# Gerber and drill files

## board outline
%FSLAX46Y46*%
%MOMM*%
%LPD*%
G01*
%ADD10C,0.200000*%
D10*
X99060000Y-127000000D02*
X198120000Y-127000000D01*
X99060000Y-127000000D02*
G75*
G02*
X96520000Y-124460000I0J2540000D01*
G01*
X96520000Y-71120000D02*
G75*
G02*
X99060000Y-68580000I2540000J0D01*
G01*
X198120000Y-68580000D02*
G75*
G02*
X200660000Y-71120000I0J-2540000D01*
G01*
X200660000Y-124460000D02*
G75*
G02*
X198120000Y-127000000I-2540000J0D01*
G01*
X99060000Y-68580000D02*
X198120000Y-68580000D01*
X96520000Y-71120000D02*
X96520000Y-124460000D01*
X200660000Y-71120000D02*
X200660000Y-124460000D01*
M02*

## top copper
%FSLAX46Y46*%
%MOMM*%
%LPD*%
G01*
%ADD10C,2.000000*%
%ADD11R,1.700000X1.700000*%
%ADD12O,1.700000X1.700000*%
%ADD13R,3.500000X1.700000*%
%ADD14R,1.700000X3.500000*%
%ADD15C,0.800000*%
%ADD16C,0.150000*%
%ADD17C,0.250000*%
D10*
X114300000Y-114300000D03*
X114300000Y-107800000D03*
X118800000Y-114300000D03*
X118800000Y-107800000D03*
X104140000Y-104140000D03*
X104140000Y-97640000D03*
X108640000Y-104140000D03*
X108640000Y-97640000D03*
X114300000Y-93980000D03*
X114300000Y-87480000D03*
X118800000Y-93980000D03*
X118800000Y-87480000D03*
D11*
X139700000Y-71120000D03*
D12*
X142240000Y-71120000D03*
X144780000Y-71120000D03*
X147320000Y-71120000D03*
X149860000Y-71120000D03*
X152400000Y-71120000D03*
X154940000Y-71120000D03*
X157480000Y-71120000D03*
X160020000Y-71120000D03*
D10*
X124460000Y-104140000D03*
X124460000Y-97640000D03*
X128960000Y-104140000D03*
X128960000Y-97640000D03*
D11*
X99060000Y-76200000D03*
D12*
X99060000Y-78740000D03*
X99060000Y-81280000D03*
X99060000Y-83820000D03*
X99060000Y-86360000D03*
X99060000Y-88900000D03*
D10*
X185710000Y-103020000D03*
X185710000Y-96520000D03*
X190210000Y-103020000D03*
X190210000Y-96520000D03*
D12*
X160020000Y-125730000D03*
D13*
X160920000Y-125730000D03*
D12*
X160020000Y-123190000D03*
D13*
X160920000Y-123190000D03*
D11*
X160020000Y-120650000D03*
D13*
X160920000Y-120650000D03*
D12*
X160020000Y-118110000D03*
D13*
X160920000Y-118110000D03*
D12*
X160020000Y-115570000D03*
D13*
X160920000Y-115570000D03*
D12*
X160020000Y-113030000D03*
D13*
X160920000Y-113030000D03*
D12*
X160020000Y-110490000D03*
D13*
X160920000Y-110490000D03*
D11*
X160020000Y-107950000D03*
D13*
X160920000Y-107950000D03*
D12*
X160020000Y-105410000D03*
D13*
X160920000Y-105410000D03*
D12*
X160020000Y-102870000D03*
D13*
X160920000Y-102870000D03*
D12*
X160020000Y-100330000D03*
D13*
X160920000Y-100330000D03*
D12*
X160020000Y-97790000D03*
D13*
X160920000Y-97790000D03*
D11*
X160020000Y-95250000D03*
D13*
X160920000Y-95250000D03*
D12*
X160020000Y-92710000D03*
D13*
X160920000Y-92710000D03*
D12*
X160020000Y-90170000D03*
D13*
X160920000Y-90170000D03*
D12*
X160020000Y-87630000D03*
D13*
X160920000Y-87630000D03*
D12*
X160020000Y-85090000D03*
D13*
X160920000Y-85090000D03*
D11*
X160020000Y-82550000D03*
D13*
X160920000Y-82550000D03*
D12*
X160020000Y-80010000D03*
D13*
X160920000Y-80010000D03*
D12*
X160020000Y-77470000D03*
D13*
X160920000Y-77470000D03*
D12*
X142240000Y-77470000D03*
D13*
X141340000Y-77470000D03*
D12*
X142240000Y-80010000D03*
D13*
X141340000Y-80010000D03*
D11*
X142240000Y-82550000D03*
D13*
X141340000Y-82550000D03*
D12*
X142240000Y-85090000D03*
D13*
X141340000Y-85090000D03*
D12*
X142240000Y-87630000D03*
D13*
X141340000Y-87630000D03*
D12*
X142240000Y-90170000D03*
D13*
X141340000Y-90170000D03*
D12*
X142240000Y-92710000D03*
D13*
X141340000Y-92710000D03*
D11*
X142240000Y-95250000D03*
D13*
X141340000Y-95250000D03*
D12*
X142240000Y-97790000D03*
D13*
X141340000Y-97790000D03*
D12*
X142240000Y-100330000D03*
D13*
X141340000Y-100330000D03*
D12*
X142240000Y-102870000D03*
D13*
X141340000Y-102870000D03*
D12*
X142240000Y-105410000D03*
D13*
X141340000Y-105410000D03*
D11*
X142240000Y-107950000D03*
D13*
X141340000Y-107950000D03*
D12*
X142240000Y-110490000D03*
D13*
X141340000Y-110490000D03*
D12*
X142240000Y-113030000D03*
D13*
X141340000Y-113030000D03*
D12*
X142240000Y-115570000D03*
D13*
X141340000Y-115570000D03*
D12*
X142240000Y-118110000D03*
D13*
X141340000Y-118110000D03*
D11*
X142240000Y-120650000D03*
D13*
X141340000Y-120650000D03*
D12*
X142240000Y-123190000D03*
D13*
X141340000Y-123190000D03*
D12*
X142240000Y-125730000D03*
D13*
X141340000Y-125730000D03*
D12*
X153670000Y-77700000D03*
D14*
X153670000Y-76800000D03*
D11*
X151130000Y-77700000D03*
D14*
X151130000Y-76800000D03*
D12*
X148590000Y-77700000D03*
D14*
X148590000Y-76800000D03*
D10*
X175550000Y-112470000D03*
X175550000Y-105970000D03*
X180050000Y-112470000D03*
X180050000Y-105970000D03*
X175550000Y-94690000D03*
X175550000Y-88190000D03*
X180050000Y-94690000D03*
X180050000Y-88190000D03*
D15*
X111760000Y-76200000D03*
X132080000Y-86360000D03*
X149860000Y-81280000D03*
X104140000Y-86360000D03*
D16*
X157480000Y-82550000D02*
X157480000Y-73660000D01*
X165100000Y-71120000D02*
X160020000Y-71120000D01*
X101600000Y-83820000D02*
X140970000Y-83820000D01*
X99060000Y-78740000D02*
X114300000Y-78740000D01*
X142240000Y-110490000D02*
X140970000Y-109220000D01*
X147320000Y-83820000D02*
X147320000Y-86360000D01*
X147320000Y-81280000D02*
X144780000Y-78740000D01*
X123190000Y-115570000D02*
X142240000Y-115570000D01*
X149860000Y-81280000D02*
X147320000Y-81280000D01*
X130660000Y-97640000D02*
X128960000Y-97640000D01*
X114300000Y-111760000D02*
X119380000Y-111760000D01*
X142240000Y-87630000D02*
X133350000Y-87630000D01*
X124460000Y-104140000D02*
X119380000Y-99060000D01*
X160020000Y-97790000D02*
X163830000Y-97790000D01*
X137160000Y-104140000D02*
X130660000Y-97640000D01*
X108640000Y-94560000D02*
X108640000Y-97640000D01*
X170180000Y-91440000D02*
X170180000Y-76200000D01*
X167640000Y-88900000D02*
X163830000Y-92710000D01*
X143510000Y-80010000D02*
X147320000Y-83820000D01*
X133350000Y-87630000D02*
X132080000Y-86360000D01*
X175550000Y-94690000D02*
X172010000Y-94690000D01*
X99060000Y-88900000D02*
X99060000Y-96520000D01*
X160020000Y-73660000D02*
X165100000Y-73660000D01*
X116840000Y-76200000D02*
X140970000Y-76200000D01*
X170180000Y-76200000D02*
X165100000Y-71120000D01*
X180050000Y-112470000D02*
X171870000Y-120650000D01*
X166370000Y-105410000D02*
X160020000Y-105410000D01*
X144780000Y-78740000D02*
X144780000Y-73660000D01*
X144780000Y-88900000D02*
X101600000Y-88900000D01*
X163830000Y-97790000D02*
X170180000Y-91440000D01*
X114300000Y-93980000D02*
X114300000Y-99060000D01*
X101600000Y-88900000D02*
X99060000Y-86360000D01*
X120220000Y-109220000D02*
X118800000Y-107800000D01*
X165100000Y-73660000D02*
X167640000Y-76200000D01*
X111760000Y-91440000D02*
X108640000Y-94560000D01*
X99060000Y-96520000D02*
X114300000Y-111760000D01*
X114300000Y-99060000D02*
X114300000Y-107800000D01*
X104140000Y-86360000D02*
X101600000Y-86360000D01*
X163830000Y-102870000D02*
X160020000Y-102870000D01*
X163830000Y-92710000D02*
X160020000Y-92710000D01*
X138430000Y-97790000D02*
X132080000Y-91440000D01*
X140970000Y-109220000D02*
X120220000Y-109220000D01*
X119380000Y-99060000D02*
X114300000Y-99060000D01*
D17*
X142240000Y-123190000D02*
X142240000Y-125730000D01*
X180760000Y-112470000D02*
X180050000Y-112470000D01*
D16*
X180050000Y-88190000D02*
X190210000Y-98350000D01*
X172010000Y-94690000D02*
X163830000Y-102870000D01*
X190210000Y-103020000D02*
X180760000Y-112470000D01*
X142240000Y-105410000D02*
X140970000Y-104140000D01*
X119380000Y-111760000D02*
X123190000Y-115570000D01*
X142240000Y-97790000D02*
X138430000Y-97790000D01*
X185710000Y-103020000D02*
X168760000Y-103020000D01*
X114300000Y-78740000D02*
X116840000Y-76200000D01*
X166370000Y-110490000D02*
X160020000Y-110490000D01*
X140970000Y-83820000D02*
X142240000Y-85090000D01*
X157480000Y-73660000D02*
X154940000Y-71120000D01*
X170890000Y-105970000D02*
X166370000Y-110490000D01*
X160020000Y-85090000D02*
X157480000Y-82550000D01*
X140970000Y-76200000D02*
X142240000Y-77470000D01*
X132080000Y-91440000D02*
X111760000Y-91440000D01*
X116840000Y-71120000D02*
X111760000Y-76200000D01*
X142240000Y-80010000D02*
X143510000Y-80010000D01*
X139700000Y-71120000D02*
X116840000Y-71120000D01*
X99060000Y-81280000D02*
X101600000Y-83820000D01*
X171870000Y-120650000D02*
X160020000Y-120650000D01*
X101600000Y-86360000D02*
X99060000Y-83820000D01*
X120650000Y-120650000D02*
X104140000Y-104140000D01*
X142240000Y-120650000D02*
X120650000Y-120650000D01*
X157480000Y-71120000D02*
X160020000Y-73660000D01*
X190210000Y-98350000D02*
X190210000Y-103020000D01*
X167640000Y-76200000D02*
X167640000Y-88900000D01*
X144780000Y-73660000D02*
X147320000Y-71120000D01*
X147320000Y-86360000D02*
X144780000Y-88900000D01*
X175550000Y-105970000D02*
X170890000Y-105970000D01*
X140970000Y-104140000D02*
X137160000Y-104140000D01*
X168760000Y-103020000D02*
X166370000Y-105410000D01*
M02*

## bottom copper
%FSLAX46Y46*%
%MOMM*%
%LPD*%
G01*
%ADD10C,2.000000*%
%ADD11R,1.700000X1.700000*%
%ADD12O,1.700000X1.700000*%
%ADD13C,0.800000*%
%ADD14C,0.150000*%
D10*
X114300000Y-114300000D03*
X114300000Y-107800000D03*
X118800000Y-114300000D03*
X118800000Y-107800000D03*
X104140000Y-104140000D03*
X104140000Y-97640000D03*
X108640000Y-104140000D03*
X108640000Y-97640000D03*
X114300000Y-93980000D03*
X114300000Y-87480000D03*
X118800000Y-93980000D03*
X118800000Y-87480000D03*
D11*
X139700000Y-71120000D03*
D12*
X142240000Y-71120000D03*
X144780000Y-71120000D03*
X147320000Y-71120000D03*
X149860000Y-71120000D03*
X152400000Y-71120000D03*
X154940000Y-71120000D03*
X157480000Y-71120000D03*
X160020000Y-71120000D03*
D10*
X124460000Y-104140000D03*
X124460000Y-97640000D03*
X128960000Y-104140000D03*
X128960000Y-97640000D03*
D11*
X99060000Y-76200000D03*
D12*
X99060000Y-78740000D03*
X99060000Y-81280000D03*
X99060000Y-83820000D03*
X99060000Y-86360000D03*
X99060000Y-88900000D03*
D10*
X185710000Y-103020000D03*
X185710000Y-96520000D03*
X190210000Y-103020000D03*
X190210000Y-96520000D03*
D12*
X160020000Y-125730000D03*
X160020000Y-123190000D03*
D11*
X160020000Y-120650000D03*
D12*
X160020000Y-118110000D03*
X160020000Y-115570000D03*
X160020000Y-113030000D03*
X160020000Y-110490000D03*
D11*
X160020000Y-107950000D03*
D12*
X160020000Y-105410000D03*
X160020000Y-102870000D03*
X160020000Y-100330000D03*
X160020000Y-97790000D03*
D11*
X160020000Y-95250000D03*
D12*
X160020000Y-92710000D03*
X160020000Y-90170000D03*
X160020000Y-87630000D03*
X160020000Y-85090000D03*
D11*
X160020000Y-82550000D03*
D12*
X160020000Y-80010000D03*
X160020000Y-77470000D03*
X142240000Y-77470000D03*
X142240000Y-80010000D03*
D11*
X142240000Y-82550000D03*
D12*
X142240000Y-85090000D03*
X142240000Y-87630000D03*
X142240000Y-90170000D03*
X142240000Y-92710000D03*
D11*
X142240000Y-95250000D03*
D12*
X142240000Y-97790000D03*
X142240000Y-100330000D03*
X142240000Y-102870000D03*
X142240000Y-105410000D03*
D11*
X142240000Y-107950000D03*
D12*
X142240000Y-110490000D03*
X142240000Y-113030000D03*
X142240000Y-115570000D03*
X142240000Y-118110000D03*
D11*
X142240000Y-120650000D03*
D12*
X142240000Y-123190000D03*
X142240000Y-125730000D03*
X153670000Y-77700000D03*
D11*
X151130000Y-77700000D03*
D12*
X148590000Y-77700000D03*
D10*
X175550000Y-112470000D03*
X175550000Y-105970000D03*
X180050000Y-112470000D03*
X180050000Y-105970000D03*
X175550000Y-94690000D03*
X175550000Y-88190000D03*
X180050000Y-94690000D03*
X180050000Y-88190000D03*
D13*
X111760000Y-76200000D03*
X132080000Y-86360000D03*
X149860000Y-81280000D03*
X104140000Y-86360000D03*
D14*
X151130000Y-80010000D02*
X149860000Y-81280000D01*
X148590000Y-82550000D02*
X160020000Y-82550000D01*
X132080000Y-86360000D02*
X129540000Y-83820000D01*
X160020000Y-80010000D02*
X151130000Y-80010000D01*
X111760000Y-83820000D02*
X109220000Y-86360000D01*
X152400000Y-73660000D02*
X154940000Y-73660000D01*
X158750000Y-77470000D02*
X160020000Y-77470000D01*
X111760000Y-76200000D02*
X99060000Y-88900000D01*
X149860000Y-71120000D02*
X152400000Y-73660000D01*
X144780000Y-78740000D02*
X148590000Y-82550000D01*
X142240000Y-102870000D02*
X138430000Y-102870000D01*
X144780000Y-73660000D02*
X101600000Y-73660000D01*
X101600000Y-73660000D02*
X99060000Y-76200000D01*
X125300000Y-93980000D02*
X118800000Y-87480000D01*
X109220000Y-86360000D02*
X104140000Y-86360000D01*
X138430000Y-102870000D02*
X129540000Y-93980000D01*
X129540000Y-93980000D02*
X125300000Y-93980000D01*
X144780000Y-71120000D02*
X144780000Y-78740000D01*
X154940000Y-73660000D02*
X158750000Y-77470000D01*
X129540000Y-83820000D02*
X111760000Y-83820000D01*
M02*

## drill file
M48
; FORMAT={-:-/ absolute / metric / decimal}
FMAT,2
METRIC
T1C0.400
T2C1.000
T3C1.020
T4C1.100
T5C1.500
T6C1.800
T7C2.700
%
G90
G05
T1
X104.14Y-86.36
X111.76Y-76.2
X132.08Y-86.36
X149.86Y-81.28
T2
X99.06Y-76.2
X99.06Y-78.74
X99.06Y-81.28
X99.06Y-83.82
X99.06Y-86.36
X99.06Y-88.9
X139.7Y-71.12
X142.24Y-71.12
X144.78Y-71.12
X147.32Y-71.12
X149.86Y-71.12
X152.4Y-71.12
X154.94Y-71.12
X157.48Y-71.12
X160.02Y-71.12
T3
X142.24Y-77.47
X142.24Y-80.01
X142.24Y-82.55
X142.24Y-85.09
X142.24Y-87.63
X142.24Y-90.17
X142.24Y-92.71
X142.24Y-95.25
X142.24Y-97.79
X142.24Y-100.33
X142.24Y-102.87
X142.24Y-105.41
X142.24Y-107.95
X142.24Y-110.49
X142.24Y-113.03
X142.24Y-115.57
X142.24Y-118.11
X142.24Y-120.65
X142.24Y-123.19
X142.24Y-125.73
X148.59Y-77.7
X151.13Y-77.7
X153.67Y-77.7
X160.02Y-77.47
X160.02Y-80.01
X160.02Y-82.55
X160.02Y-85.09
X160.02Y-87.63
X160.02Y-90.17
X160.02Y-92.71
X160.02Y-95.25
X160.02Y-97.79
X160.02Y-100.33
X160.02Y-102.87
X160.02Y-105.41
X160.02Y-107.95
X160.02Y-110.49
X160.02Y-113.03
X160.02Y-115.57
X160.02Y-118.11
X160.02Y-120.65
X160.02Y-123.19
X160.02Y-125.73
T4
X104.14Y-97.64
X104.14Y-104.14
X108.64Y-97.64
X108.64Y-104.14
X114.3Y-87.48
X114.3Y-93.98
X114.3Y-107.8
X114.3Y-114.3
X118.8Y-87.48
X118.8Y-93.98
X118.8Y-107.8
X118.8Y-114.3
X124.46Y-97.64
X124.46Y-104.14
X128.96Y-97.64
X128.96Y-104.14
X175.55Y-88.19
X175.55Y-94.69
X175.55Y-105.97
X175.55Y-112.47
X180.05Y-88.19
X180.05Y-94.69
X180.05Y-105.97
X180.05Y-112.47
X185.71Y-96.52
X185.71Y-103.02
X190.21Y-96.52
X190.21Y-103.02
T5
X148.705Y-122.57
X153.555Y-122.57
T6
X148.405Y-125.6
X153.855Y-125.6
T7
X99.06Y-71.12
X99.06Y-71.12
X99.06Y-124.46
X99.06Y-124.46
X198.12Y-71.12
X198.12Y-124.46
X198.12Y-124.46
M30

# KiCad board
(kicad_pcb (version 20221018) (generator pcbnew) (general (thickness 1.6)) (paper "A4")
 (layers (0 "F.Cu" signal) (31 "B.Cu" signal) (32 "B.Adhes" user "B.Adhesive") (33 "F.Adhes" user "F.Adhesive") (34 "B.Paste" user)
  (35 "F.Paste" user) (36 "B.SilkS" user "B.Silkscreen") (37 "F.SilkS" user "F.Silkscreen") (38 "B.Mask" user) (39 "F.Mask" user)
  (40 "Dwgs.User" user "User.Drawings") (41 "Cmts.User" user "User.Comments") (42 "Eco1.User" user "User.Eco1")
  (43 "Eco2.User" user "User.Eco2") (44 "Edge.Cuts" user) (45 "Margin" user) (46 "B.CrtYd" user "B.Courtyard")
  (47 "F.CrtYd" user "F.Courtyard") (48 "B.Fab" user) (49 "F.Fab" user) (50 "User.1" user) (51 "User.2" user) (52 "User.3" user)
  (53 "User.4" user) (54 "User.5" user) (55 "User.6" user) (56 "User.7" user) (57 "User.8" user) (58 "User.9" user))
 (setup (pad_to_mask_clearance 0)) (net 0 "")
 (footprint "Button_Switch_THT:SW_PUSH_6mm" (layer "F.Cu") (at 114.3 114.3 90)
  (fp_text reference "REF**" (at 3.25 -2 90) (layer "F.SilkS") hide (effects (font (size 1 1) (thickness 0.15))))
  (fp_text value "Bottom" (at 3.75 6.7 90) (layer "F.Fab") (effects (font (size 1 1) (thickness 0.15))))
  (pad "1" thru_hole circle (at 0 0 180) (size 2 2) (drill 1.1) (layers "*.Cu" "*.Mask"))
  (pad "1" thru_hole circle (at 6.5 0 180) (size 2 2) (drill 1.1) (layers "*.Cu" "*.Mask"))
  (pad "2" thru_hole circle (at 0 4.5 180) (size 2 2) (drill 1.1) (layers "*.Cu" "*.Mask"))
  (pad "2" thru_hole circle (at 6.5 4.5 180) (size 2 2) (drill 1.1) (layers "*.Cu" "*.Mask")))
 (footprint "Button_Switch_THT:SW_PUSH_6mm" (layer "F.Cu") (at 104.14 104.14 90)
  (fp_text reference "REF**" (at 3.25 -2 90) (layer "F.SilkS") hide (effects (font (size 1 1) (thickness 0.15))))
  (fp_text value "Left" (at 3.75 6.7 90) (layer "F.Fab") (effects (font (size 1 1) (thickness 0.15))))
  (pad "1" thru_hole circle (at 0 0 180) (size 2 2) (drill 1.1) (layers "*.Cu" "*.Mask"))
  (pad "1" thru_hole circle (at 6.5 0 180) (size 2 2) (drill 1.1) (layers "*.Cu" "*.Mask"))
  (pad "2" thru_hole circle (at 0 4.5 180) (size 2 2) (drill 1.1) (layers "*.Cu" "*.Mask"))
  (pad "2" thru_hole circle (at 6.5 4.5 180) (size 2 2) (drill 1.1) (layers "*.Cu" "*.Mask")))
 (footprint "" (layer "F.Cu") (at 198.12 71.12)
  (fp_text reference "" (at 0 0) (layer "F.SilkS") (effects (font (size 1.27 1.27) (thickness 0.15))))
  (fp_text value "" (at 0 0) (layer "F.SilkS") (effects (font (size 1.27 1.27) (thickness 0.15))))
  (pad "" np_thru_hole circle (at 0 0) (size 2.7 2.7) (drill 2.7) (layers "F&B.Cu" "*.Mask")))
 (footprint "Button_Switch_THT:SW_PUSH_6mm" (layer "F.Cu") (at 114.3 93.98 90)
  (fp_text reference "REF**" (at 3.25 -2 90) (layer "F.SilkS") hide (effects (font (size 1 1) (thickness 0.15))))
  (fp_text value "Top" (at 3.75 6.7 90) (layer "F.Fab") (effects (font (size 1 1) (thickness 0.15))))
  (pad "1" thru_hole circle (at 0 0 180) (size 2 2) (drill 1.1) (layers "*.Cu" "*.Mask"))
  (pad "1" thru_hole circle (at 6.5 0 180) (size 2 2) (drill 1.1) (layers "*.Cu" "*.Mask"))
  (pad "2" thru_hole circle (at 0 4.5 180) (size 2 2) (drill 1.1) (layers "*.Cu" "*.Mask"))
  (pad "2" thru_hole circle (at 6.5 4.5 180) (size 2 2) (drill 1.1) (layers "*.Cu" "*.Mask")))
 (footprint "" (layer "F.Cu") (at 99.06 71.12)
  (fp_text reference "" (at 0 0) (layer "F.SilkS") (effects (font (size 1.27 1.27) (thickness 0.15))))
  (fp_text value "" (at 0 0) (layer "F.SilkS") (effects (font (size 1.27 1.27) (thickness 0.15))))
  (pad "" np_thru_hole circle (at 0 0) (size 2.7 2.7) (drill 2.7) (layers "F&B.Cu" "*.Mask")))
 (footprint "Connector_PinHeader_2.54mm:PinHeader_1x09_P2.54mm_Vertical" (layer "F.Cu") (at 139.7 71.12 90)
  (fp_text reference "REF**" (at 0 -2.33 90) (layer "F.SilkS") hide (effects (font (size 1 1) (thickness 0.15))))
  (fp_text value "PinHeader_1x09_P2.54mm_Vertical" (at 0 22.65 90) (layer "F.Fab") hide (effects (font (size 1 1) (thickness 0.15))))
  (pad "1" thru_hole rect (at 0 0 90) (size 1.7 1.7) (drill 1) (layers "*.Cu" "*.Mask"))
  (pad "2" thru_hole oval (at 0 2.54 90) (size 1.7 1.7) (drill 1) (layers "*.Cu" "*.Mask"))
  (pad "3" thru_hole oval (at 0 5.08 90) (size 1.7 1.7) (drill 1) (layers "*.Cu" "*.Mask"))
  (pad "4" thru_hole oval (at 0 7.62 90) (size 1.7 1.7) (drill 1) (layers "*.Cu" "*.Mask"))
  (pad "5" thru_hole oval (at 0 10.16 90) (size 1.7 1.7) (drill 1) (layers "*.Cu" "*.Mask"))
  (pad "6" thru_hole oval (at 0 12.7 90) (size 1.7 1.7) (drill 1) (layers "*.Cu" "*.Mask"))
  (pad "7" thru_hole oval (at 0 15.24 90) (size 1.7 1.7) (drill 1) (layers "*.Cu" "*.Mask"))
  (pad "8" thru_hole oval (at 0 17.78 90) (size 1.7 1.7) (drill 1) (layers "*.Cu" "*.Mask"))
  (pad "9" thru_hole oval (at 0 20.32 90) (size 1.7 1.7) (drill 1) (layers "*.Cu" "*.Mask")))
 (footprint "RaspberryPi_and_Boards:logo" (layer "F.Cu") (at 190.5 76.2)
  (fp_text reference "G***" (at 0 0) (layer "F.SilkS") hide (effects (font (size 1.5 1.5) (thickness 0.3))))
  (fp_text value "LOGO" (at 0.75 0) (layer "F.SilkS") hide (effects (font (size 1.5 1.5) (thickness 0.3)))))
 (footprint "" (layer "F.Cu") (at 198.12 124.46)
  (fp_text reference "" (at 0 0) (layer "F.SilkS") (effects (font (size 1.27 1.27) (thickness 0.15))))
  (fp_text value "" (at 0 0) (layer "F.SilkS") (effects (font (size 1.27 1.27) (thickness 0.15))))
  (pad "" np_thru_hole circle (at 0 0) (size 2.7 2.7) (drill 2.7) (layers "F&B.Cu" "*.Mask")))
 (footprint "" (layer "F.Cu") (at 198.12 124.46)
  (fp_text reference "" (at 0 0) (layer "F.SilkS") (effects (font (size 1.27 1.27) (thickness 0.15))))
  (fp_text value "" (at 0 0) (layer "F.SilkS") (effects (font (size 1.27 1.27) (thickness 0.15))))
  (pad "" np_thru_hole circle (at 0 0) (size 2.7 2.7) (drill 2.7) (layers "F&B.Cu" "*.Mask")))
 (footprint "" (layer "F.Cu") (at 99.06 124.46)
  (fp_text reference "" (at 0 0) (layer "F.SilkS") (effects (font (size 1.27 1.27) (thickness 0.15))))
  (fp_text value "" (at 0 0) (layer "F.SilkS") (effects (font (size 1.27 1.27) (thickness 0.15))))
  (pad "" np_thru_hole circle (at 0 0) (size 2.7 2.7) (drill 2.7) (layers "F&B.Cu" "*.Mask")))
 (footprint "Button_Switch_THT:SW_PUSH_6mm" (layer "F.Cu") (at 124.46 104.14 90)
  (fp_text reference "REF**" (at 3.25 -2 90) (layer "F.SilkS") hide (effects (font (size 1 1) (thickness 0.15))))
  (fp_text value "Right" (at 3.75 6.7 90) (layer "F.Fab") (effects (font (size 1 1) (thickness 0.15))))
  (pad "1" thru_hole circle (at 0 0 180) (size 2 2) (drill 1.1) (layers "*.Cu" "*.Mask"))
  (pad "1" thru_hole circle (at 6.5 0 180) (size 2 2) (drill 1.1) (layers "*.Cu" "*.Mask"))
  (pad "2" thru_hole circle (at 0 4.5 180) (size 2 2) (drill 1.1) (layers "*.Cu" "*.Mask"))
  (pad "2" thru_hole circle (at 6.5 4.5 180) (size 2 2) (drill 1.1) (layers "*.Cu" "*.Mask")))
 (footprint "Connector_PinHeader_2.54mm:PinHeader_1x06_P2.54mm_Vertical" (layer "F.Cu") (at 99.06 76.2)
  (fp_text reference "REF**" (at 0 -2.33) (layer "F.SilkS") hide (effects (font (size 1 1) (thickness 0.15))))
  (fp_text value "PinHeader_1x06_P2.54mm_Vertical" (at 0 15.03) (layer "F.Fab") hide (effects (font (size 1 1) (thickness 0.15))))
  (pad "1" thru_hole rect (at 0 0) (size 1.7 1.7) (drill 1) (layers "*.Cu" "*.Mask"))
  (pad "2" thru_hole oval (at 0 2.54) (size 1.7 1.7) (drill 1) (layers "*.Cu" "*.Mask"))
  (pad "3" thru_hole oval (at 0 5.08) (size 1.7 1.7) (drill 1) (layers "*.Cu" "*.Mask"))
  (pad "4" thru_hole oval (at 0 7.62) (size 1.7 1.7) (drill 1) (layers "*.Cu" "*.Mask"))
  (pad "5" thru_hole oval (at 0 10.16) (size 1.7 1.7) (drill 1) (layers "*.Cu" "*.Mask"))
  (pad "6" thru_hole oval (at 0 12.7) (size 1.7 1.7) (drill 1) (layers "*.Cu" "*.Mask")))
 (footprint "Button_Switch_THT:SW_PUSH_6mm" (layer "F.Cu") (at 185.71 103.02 90)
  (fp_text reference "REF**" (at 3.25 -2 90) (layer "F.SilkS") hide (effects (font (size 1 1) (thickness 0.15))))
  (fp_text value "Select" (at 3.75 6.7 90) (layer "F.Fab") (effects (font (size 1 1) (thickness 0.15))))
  (pad "1" thru_hole circle (at 0 0 180) (size 2 2) (drill 1.1) (layers "*.Cu" "*.Mask"))
  (pad "1" thru_hole circle (at 6.5 0 180) (size 2 2) (drill 1.1) (layers "*.Cu" "*.Mask"))
  (pad "2" thru_hole circle (at 0 4.5 180) (size 2 2) (drill 1.1) (layers "*.Cu" "*.Mask"))
  (pad "2" thru_hole circle (at 6.5 4.5 180) (size 2 2) (drill 1.1) (layers "*.Cu" "*.Mask")))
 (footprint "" (layer "F.Cu") (at 99.06 124.46)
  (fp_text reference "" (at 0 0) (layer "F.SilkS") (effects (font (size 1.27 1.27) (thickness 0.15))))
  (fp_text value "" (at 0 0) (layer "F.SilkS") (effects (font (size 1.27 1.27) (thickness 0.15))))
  (pad "" np_thru_hole circle (at 0 0) (size 2.7 2.7) (drill 2.7) (layers "F&B.Cu" "*.Mask")))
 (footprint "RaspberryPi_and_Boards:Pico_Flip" (layer "F.Cu") (at 151.13 101.6 180)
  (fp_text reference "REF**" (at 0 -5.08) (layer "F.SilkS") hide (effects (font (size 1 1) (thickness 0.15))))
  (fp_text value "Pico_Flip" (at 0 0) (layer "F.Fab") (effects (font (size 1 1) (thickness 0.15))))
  (pad "" np_thru_hole oval (at -2.725 -24 180) (size 1.8 1.8) (drill 1.8) (layers "*.Cu" "*.Mask"))
  (pad "" np_thru_hole oval (at -2.425 -20.97 180) (size 1.5 1.5) (drill 1.5) (layers "*.Cu" "*.Mask"))
  (pad "" np_thru_hole oval (at 2.425 -20.97 180) (size 1.5 1.5) (drill 1.5) (layers "*.Cu" "*.Mask"))
  (pad "" np_thru_hole oval (at 2.725 -24 180) (size 1.8 1.8) (drill 1.8) (layers "*.Cu" "*.Mask"))
  (pad "1" thru_hole oval (at -8.89 -24.13 180) (size 1.7 1.7) (drill 1.02) (layers "*.Cu" "*.Mask"))
  (pad "1" smd rect (at -8.89 -24.13 180) (size 3.5 1.7) (drill (offset -0.9 0)) (layers "F.Cu" "F.Mask"))
  (pad "2" thru_hole oval (at -8.89 -21.59 180) (size 1.7 1.7) (drill 1.02) (layers "*.Cu" "*.Mask"))
  (pad "2" smd rect (at -8.89 -21.59 180) (size 3.5 1.7) (drill (offset -0.9 0)) (layers "F.Cu" "F.Mask"))
  (pad "3" thru_hole rect (at -8.89 -19.05 180) (size 1.7 1.7) (drill 1.02) (layers "*.Cu" "*.Mask"))
  (pad "3" smd rect (at -8.89 -19.05 180) (size 3.5 1.7) (drill (offset -0.9 0)) (layers "F.Cu" "F.Mask"))
  (pad "4" thru_hole oval (at -8.89 -16.51 180) (size 1.7 1.7) (drill 1.02) (layers "*.Cu" "*.Mask"))
  (pad "4" smd rect (at -8.89 -16.51 180) (size 3.5 1.7) (drill (offset -0.9 0)) (layers "F.Cu" "F.Mask"))
  (pad "5" thru_hole oval (at -8.89 -13.97 180) (size 1.7 1.7) (drill 1.02) (layers "*.Cu" "*.Mask"))
  (pad "5" smd rect (at -8.89 -13.97 180) (size 3.5 1.7) (drill (offset -0.9 0)) (layers "F.Cu" "F.Mask"))
  (pad "6" thru_hole oval (at -8.89 -11.43 180) (size 1.7 1.7) (drill 1.02) (layers "*.Cu" "*.Mask"))
  (pad "6" smd rect (at -8.89 -11.43 180) (size 3.5 1.7) (drill (offset -0.9 0)) (layers "F.Cu" "F.Mask"))
  (pad "7" thru_hole oval (at -8.89 -8.89 180) (size 1.7 1.7) (drill 1.02) (layers "*.Cu" "*.Mask"))
  (pad "7" smd rect (at -8.89 -8.89 180) (size 3.5 1.7) (drill (offset -0.9 0)) (layers "F.Cu" "F.Mask"))
  (pad "8" thru_hole rect (at -8.89 -6.35 180) (size 1.7 1.7) (drill 1.02) (layers "*.Cu" "*.Mask"))
  (pad "8" smd rect (at -8.89 -6.35 180) (size 3.5 1.7) (drill (offset -0.9 0)) (layers "F.Cu" "F.Mask"))
  (pad "9" thru_hole oval (at -8.89 -3.81 180) (size 1.7 1.7) (drill 1.02) (layers "*.Cu" "*.Mask"))
  (pad "9" smd rect (at -8.89 -3.81 180) (size 3.5 1.7) (drill (offset -0.9 0)) (layers "F.Cu" "F.Mask"))
  (pad "10" thru_hole oval (at -8.89 -1.27 180) (size 1.7 1.7) (drill 1.02) (layers "*.Cu" "*.Mask"))
  (pad "10" smd rect (at -8.89 -1.27 180) (size 3.5 1.7) (drill (offset -0.9 0)) (layers "F.Cu" "F.Mask"))
  (pad "11" thru_hole oval (at -8.89 1.27 180) (size 1.7 1.7) (drill 1.02) (layers "*.Cu" "*.Mask"))
  (pad "11" smd rect (at -8.89 1.27 180) (size 3.5 1.7) (drill (offset -0.9 0)) (layers "F.Cu" "F.Mask"))
  (pad "12" thru_hole oval (at -8.89 3.81 180) (size 1.7 1.7) (drill 1.02) (layers "*.Cu" "*.Mask"))
  (pad "12" smd rect (at -8.89 3.81 180) (size 3.5 1.7) (drill (offset -0.9 0)) (layers "F.Cu" "F.Mask"))
  (pad "13" thru_hole rect (at -8.89 6.35 180) (size 1.7 1.7) (drill 1.02) (layers "*.Cu" "*.Mask"))
  (pad "13" smd rect (at -8.89 6.35 180) (size 3.5 1.7) (drill (offset -0.9 0)) (layers "F.Cu" "F.Mask"))
  (pad "14" thru_hole oval (at -8.89 8.89 180) (size 1.7 1.7) (drill 1.02) (layers "*.Cu" "*.Mask"))
  (pad "14" smd rect (at -8.89 8.89 180) (size 3.5 1.7) (drill (offset -0.9 0)) (layers "F.Cu" "F.Mask"))
  (pad "15" thru_hole oval (at -8.89 11.43 180) (size 1.7 1.7) (drill 1.02) (layers "*.Cu" "*.Mask"))
  (pad "15" smd rect (at -8.89 11.43 180) (size 3.5 1.7) (drill (offset -0.9 0)) (layers "F.Cu" "F.Mask"))
  (pad "16" thru_hole oval (at -8.89 13.97 180) (size 1.7 1.7) (drill 1.02) (layers "*.Cu" "*.Mask"))
  (pad "16" smd rect (at -8.89 13.97 180) (size 3.5 1.7) (drill (offset -0.9 0)) (layers "F.Cu" "F.Mask"))
  (pad "17" thru_hole oval (at -8.89 16.51 180) (size 1.7 1.7) (drill 1.02) (layers "*.Cu" "*.Mask"))
  (pad "17" smd rect (at -8.89 16.51 180) (size 3.5 1.7) (drill (offset -0.9 0)) (layers "F.Cu" "F.Mask"))
  (pad "18" thru_hole rect (at -8.89 19.05 180) (size 1.7 1.7) (drill 1.02) (layers "*.Cu" "*.Mask"))
  (pad "18" smd rect (at -8.89 19.05 180) (size 3.5 1.7) (drill (offset -0.9 0)) (layers "F.Cu" "F.Mask"))
  (pad "19" thru_hole oval (at -8.89 21.59 180) (size 1.7 1.7) (drill 1.02) (layers "*.Cu" "*.Mask"))
  (pad "19" smd rect (at -8.89 21.59 180) (size 3.5 1.7) (drill (offset -0.9 0)) (layers "F.Cu" "F.Mask"))
  (pad "20" thru_hole oval (at -8.89 24.13 180) (size 1.7 1.7) (drill 1.02) (layers "*.Cu" "*.Mask"))
  (pad "20" smd rect (at -8.89 24.13 180) (size 3.5 1.7) (drill (offset -0.9 0)) (layers "F.Cu" "F.Mask"))
  (pad "21" thru_hole oval (at 8.89 24.13 180) (size 1.7 1.7) (drill 1.02) (layers "*.Cu" "*.Mask"))
  (pad "21" smd rect (at 8.89 24.13 180) (size 3.5 1.7) (drill (offset 0.9 0)) (layers "F.Cu" "F.Mask"))
  (pad "22" thru_hole oval (at 8.89 21.59 180) (size 1.7 1.7) (drill 1.02) (layers "*.Cu" "*.Mask"))
  (pad "22" smd rect (at 8.89 21.59 180) (size 3.5 1.7) (drill (offset 0.9 0)) (layers "F.Cu" "F.Mask"))
  (pad "23" thru_hole rect (at 8.89 19.05 180) (size 1.7 1.7) (drill 1.02) (layers "*.Cu" "*.Mask"))
  (pad "23" smd rect (at 8.89 19.05 180) (size 3.5 1.7) (drill (offset 0.9 0)) (layers "F.Cu" "F.Mask"))
  (pad "24" thru_hole oval (at 8.89 16.51 180) (size 1.7 1.7) (drill 1.02) (layers "*.Cu" "*.Mask"))
  (pad "24" smd rect (at 8.89 16.51 180) (size 3.5 1.7) (drill (offset 0.9 0)) (layers "F.Cu" "F.Mask"))
  (pad "25" thru_hole oval (at 8.89 13.97 180) (size 1.7 1.7) (drill 1.02) (layers "*.Cu" "*.Mask"))
  (pad "25" smd rect (at 8.89 13.97 180) (size 3.5 1.7) (drill (offset 0.9 0)) (layers "F.Cu" "F.Mask"))
  (pad "26" thru_hole oval (at 8.89 11.43 180) (size 1.7 1.7) (drill 1.02) (layers "*.Cu" "*.Mask"))
  (pad "26" smd rect (at 8.89 11.43 180) (size 3.5 1.7) (drill (offset 0.9 0)) (layers "F.Cu" "F.Mask"))
  (pad "27" thru_hole oval (at 8.89 8.89 180) (size 1.7 1.7) (drill 1.02) (layers "*.Cu" "*.Mask"))
  (pad "27" smd rect (at 8.89 8.89 180) (size 3.5 1.7) (drill (offset 0.9 0)) (layers "F.Cu" "F.Mask"))
  (pad "28" thru_hole rect (at 8.89 6.35 180) (size 1.7 1.7) (drill 1.02) (layers "*.Cu" "*.Mask"))
  (pad "28" smd rect (at 8.89 6.35 180) (size 3.5 1.7) (drill (offset 0.9 0)) (layers "F.Cu" "F.Mask"))
  (pad "29" thru_hole oval (at 8.89 3.81 180) (size 1.7 1.7) (drill 1.02) (layers "*.Cu" "*.Mask"))
  (pad "29" smd rect (at 8.89 3.81 180) (size 3.5 1.7) (drill (offset 0.9 0)) (layers "F.Cu" "F.Mask"))
  (pad "30" thru_hole oval (at 8.89 1.27 180) (size 1.7 1.7) (drill 1.02) (layers "*.Cu" "*.Mask"))
  (pad "30" smd rect (at 8.89 1.27 180) (size 3.5 1.7) (drill (offset 0.9 0)) (layers "F.Cu" "F.Mask"))
  (pad "31" thru_hole oval (at 8.89 -1.27 180) (size 1.7 1.7) (drill 1.02) (layers "*.Cu" "*.Mask"))
  (pad "31" smd rect (at 8.89 -1.27 180) (size 3.5 1.7) (drill (offset 0.9 0)) (layers "F.Cu" "F.Mask"))
  (pad "32" thru_hole oval (at 8.89 -3.81 180) (size 1.7 1.7) (drill 1.02) (layers "*.Cu" "*.Mask"))
  (pad "32" smd rect (at 8.89 -3.81 180) (size 3.5 1.7) (drill (offset 0.9 0)) (layers "F.Cu" "F.Mask"))
  (pad "33" thru_hole rect (at 8.89 -6.35 180) (size 1.7 1.7) (drill 1.02) (layers "*.Cu" "*.Mask"))
  (pad "33" smd rect (at 8.89 -6.35 180) (size 3.5 1.7) (drill (offset 0.9 0)) (layers "F.Cu" "F.Mask"))
  (pad "34" thru_hole oval (at 8.89 -8.89 180) (size 1.7 1.7) (drill 1.02) (layers "*.Cu" "*.Mask"))
  (pad "34" smd rect (at 8.89 -8.89 180) (size 3.5 1.7) (drill (offset 0.9 0)) (layers "F.Cu" "F.Mask"))
  (pad "35" thru_hole oval (at 8.89 -11.43 180) (size 1.7 1.7) (drill 1.02) (layers "*.Cu" "*.Mask"))
  (pad "35" smd rect (at 8.89 -11.43 180) (size 3.5 1.7) (drill (offset 0.9 0)) (layers "F.Cu" "F.Mask"))
  (pad "36" thru_hole oval (at 8.89 -13.97 180) (size 1.7 1.7) (drill 1.02) (layers "*.Cu" "*.Mask"))
  (pad "36" smd rect (at 8.89 -13.97 180) (size 3.5 1.7) (drill (offset 0.9 0)) (layers "F.Cu" "F.Mask"))
  (pad "37" thru_hole oval (at 8.89 -16.51 180) (size 1.7 1.7) (drill 1.02) (layers "*.Cu" "*.Mask"))
  (pad "37" smd rect (at 8.89 -16.51 180) (size 3.5 1.7) (drill (offset 0.9 0)) (layers "F.Cu" "F.Mask"))
  (pad "38" thru_hole rect (at 8.89 -19.05 180) (size 1.7 1.7) (drill 1.02) (layers "*.Cu" "*.Mask"))
  (pad "38" smd rect (at 8.89 -19.05 180) (size 3.5 1.7) (drill (offset 0.9 0)) (layers "F.Cu" "F.Mask"))
  (pad "39" thru_hole oval (at 8.89 -21.59 180) (size 1.7 1.7) (drill 1.02) (layers "*.Cu" "*.Mask"))
  (pad "39" smd rect (at 8.89 -21.59 180) (size 3.5 1.7) (drill (offset 0.9 0)) (layers "F.Cu" "F.Mask"))
  (pad "40" thru_hole oval (at 8.89 -24.13 180) (size 1.7 1.7) (drill 1.02) (layers "*.Cu" "*.Mask"))
  (pad "40" smd rect (at 8.89 -24.13 180) (size 3.5 1.7) (drill (offset 0.9 0)) (layers "F.Cu" "F.Mask"))
  (pad "41" thru_hole oval (at -2.54 23.9 180) (size 1.7 1.7) (drill 1.02) (layers "*.Cu" "*.Mask"))
  (pad "41" smd rect (at -2.54 23.9 270) (size 3.5 1.7) (drill (offset -0.9 0)) (layers "F.Cu" "F.Mask"))
  (pad "42" thru_hole rect (at 0 23.9 180) (size 1.7 1.7) (drill 1.02) (layers "*.Cu" "*.Mask"))
  (pad "42" smd rect (at 0 23.9 270) (size 3.5 1.7) (drill (offset -0.9 0)) (layers "F.Cu" "F.Mask"))
  (pad "43" thru_hole oval (at 2.54 23.9 180) (size 1.7 1.7) (drill 1.02) (layers "*.Cu" "*.Mask"))
  (pad "43" smd rect (at 2.54 23.9 270) (size 3.5 1.7) (drill (offset -0.9 0)) (layers "F.Cu" "F.Mask")))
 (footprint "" (layer "F.Cu") (at 99.06 71.12)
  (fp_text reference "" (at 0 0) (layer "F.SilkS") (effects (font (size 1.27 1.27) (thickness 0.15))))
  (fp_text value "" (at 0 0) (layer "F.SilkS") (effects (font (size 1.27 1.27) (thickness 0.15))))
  (pad "" np_thru_hole circle (at 0 0) (size 2.7 2.7) (drill 2.7) (layers "F&B.Cu" "*.Mask")))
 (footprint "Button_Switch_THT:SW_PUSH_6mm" (layer "F.Cu") (at 175.55 112.47 90)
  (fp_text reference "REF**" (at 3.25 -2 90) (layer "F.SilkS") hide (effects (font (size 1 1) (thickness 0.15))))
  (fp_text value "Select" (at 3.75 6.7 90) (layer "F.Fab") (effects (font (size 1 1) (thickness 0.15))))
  (pad "1" thru_hole circle (at 0 0 180) (size 2 2) (drill 1.1) (layers "*.Cu" "*.Mask"))
  (pad "1" thru_hole circle (at 6.5 0 180) (size 2 2) (drill 1.1) (layers "*.Cu" "*.Mask"))
  (pad "2" thru_hole circle (at 0 4.5 180) (size 2 2) (drill 1.1) (layers "*.Cu" "*.Mask"))
  (pad "2" thru_hole circle (at 6.5 4.5 180) (size 2 2) (drill 1.1) (layers "*.Cu" "*.Mask")))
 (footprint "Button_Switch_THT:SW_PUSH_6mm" (layer "F.Cu") (at 175.55 94.69 90)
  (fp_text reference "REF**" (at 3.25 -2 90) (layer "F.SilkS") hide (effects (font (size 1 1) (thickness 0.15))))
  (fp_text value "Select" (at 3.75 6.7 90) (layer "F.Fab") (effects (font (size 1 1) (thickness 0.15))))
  (pad "1" thru_hole circle (at 0 0 180) (size 2 2) (drill 1.1) (layers "*.Cu" "*.Mask"))
  (pad "1" thru_hole circle (at 6.5 0 180) (size 2 2) (drill 1.1) (layers "*.Cu" "*.Mask"))
  (pad "2" thru_hole circle (at 0 4.5 180) (size 2 2) (drill 1.1) (layers "*.Cu" "*.Mask"))
  (pad "2" thru_hole circle (at 6.5 4.5 180) (size 2 2) (drill 1.1) (layers "*.Cu" "*.Mask")))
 (gr_line (start 99.06 127) (end 198.12 127) (stroke (width 0.2) (type default)) (layer "Edge.Cuts"))
 (gr_arc (start 99.06 127) (mid 97.263949 126.256051) (end 96.52 124.46) (stroke (width 0.2) (type default)) (layer "Edge.Cuts"))
 (gr_arc (start 96.52 71.12) (mid 97.263949 69.323949) (end 99.06 68.58) (stroke (width 0.2) (type default)) (layer "Edge.Cuts"))
 (gr_arc (start 198.12 68.58) (mid 199.916051 69.323949) (end 200.66 71.12) (stroke (width 0.2) (type default)) (layer "Edge.Cuts"))
 (gr_arc (start 200.66 124.46) (mid 199.916051 126.256051) (end 198.12 127) (stroke (width 0.2) (type default)) (layer "Edge.Cuts"))
 (gr_line (start 99.06 68.58) (end 198.12 68.58) (stroke (width 0.2) (type default)) (layer "Edge.Cuts"))
 (gr_line (start 96.52 71.12) (end 96.52 124.46) (stroke (width 0.2) (type default)) (layer "Edge.Cuts"))
 (gr_line (start 200.66 71.12) (end 200.66 124.46) (stroke (width 0.2) (type default)) (layer "Edge.Cuts"))
 (segment (start 157.48 82.55) (end 157.48 73.66) (width 0.15) (layer "F.Cu") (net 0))
 (segment (start 165.1 71.12) (end 160.02 71.12) (width 0.15) (layer "F.Cu") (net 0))
 (segment (start 101.6 83.82) (end 140.97 83.82) (width 0.15) (layer "F.Cu") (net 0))
 (segment (start 99.06 78.74) (end 114.3 78.74) (width 0.15) (layer "F.Cu") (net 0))
 (segment (start 142.24 110.49) (end 140.97 109.22) (width 0.15) (layer "F.Cu") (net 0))
 (segment (start 147.32 83.82) (end 147.32 86.36) (width 0.15) (layer "F.Cu") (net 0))
 (segment (start 147.32 81.28) (end 144.78 78.74) (width 0.15) (layer "F.Cu") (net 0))
 (segment (start 123.19 115.57) (end 142.24 115.57) (width 0.15) (layer "F.Cu") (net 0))
 (segment (start 149.86 81.28) (end 147.32 81.28) (width 0.15) (layer "F.Cu") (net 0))
 (segment (start 130.66 97.64) (end 128.96 97.64) (width 0.15) (layer "F.Cu") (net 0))
 (segment (start 114.3 111.76) (end 119.38 111.76) (width 0.15) (layer "F.Cu") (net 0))
 (segment (start 142.24 87.63) (end 133.35 87.63) (width 0.15) (layer "F.Cu") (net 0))
 (segment (start 124.46 104.14) (end 119.38 99.06) (width 0.15) (layer "F.Cu") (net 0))
 (segment (start 160.02 97.79) (end 163.83 97.79) (width 0.15) (layer "F.Cu") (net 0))
 (segment (start 137.16 104.14) (end 130.66 97.64) (width 0.15) (layer "F.Cu") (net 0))
 (segment (start 108.64 94.56) (end 108.64 97.64) (width 0.15) (layer "F.Cu") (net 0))
 (segment (start 170.18 91.44) (end 170.18 76.2) (width 0.15) (layer "F.Cu") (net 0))
 (segment (start 167.64 88.9) (end 163.83 92.71) (width 0.15) (layer "F.Cu") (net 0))
 (segment (start 143.51 80.01) (end 147.32 83.82) (width 0.15) (layer "F.Cu") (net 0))
 (segment (start 133.35 87.63) (end 132.08 86.36) (width 0.15) (layer "F.Cu") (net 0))
 (segment (start 175.55 94.69) (end 172.01 94.69) (width 0.15) (layer "F.Cu") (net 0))
 (segment (start 99.06 88.9) (end 99.06 96.52) (width 0.15) (layer "F.Cu") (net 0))
 (segment (start 160.02 73.66) (end 165.1 73.66) (width 0.15) (layer "F.Cu") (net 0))
 (segment (start 116.84 76.2) (end 140.97 76.2) (width 0.15) (layer "F.Cu") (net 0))
 (segment (start 170.18 76.2) (end 165.1 71.12) (width 0.15) (layer "F.Cu") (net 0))
 (segment (start 180.05 112.47) (end 171.87 120.65) (width 0.15) (layer "F.Cu") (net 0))
 (segment (start 166.37 105.41) (end 160.02 105.41) (width 0.15) (layer "F.Cu") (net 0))
 (segment (start 144.78 78.74) (end 144.78 73.66) (width 0.15) (layer "F.Cu") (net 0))
 (segment (start 144.78 88.9) (end 101.6 88.9) (width 0.15) (layer "F.Cu") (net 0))
 (segment (start 163.83 97.79) (end 170.18 91.44) (width 0.15) (layer "F.Cu") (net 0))
 (segment (start 114.3 93.98) (end 114.3 99.06) (width 0.15) (layer "F.Cu") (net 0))
 (segment (start 101.6 88.9) (end 99.06 86.36) (width 0.15) (layer "F.Cu") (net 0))
 (segment (start 120.22 109.22) (end 118.8 107.8) (width 0.15) (layer "F.Cu") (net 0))
 (segment (start 165.1 73.66) (end 167.64 76.2) (width 0.15) (layer "F.Cu") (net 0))
 (segment (start 111.76 91.44) (end 108.64 94.56) (width 0.15) (layer "F.Cu") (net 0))
 (segment (start 99.06 96.52) (end 114.3 111.76) (width 0.15) (layer "F.Cu") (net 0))
 (segment (start 114.3 99.06) (end 114.3 107.8) (width 0.15) (layer "F.Cu") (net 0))
 (segment (start 104.14 86.36) (end 101.6 86.36) (width 0.15) (layer "F.Cu") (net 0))
 (segment (start 163.83 102.87) (end 160.02 102.87) (width 0.15) (layer "F.Cu") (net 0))
 (segment (start 163.83 92.71) (end 160.02 92.71) (width 0.15) (layer "F.Cu") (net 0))
 (segment (start 138.43 97.79) (end 132.08 91.44) (width 0.15) (layer "F.Cu") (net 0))
 (segment (start 140.97 109.22) (end 120.22 109.22) (width 0.15) (layer "F.Cu") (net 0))
 (segment (start 119.38 99.06) (end 114.3 99.06) (width 0.15) (layer "F.Cu") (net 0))
 (segment (start 142.24 123.19) (end 142.24 125.73) (width 0.25) (layer "F.Cu") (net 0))
 (segment (start 180.76 112.47) (end 180.05 112.47) (width 0.25) (layer "F.Cu") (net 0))
 (segment (start 180.05 88.19) (end 190.21 98.35) (width 0.15) (layer "F.Cu") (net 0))
 (segment (start 172.01 94.69) (end 163.83 102.87) (width 0.15) (layer "F.Cu") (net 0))
 (segment (start 190.21 103.02) (end 180.76 112.47) (width 0.15) (layer "F.Cu") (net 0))
 (segment (start 142.24 105.41) (end 140.97 104.14) (width 0.15) (layer "F.Cu") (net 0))
 (segment (start 119.38 111.76) (end 123.19 115.57) (width 0.15) (layer "F.Cu") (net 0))
 (segment (start 142.24 97.79) (end 138.43 97.79) (width 0.15) (layer "F.Cu") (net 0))
 (segment (start 185.71 103.02) (end 168.76 103.02) (width 0.15) (layer "F.Cu") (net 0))
 (segment (start 114.3 78.74) (end 116.84 76.2) (width 0.15) (layer "F.Cu") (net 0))
 (segment (start 166.37 110.49) (end 160.02 110.49) (width 0.15) (layer "F.Cu") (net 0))
 (segment (start 140.97 83.82) (end 142.24 85.09) (width 0.15) (layer "F.Cu") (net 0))
 (segment (start 157.48 73.66) (end 154.94 71.12) (width 0.15) (layer "F.Cu") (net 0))
 (segment (start 170.89 105.97) (end 166.37 110.49) (width 0.15) (layer "F.Cu") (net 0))
 (segment (start 160.02 85.09) (end 157.48 82.55) (width 0.15) (layer "F.Cu") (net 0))
 (segment (start 140.97 76.2) (end 142.24 77.47) (width 0.15) (layer "F.Cu") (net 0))
 (segment (start 132.08 91.44) (end 111.76 91.44) (width 0.15) (layer "F.Cu") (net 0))
 (segment (start 116.84 71.12) (end 111.76 76.2) (width 0.15) (layer "F.Cu") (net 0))
 (segment (start 142.24 80.01) (end 143.51 80.01) (width 0.15) (layer "F.Cu") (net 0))
 (segment (start 139.7 71.12) (end 116.84 71.12) (width 0.15) (layer "F.Cu") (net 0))
 (segment (start 99.06 81.28) (end 101.6 83.82) (width 0.15) (layer "F.Cu") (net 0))
 (segment (start 171.87 120.65) (end 160.02 120.65) (width 0.15) (layer "F.Cu") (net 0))
 (segment (start 101.6 86.36) (end 99.06 83.82) (width 0.15) (layer "F.Cu") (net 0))
 (segment (start 120.65 120.65) (end 104.14 104.14) (width 0.15) (layer "F.Cu") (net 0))
 (segment (start 142.24 120.65) (end 120.65 120.65) (width 0.15) (layer "F.Cu") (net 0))
 (segment (start 157.48 71.12) (end 160.02 73.66) (width 0.15) (layer "F.Cu") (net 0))
 (segment (start 190.21 98.35) (end 190.21 103.02) (width 0.15) (layer "F.Cu") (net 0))
 (segment (start 167.64 76.2) (end 167.64 88.9) (width 0.15) (layer "F.Cu") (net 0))
 (segment (start 144.78 73.66) (end 147.32 71.12) (width 0.15) (layer "F.Cu") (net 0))
 (segment (start 147.32 86.36) (end 144.78 88.9) (width 0.15) (layer "F.Cu") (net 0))
 (segment (start 175.55 105.97) (end 170.89 105.97) (width 0.15) (layer "F.Cu") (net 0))
 (segment (start 140.97 104.14) (end 137.16 104.14) (width 0.15) (layer "F.Cu") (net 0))
 (segment (start 168.76 103.02) (end 166.37 105.41) (width 0.15) (layer "F.Cu") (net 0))
 (via (at 111.76 76.2) (size 0.8) (drill 0.4) (layers "F.Cu" "B.Cu") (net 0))
 (via (at 132.08 86.36) (size 0.8) (drill 0.4) (layers "F.Cu" "B.Cu") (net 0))
 (via (at 149.86 81.28) (size 0.8) (drill 0.4) (layers "F.Cu" "B.Cu") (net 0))
 (via (at 104.14 86.36) (size 0.8) (drill 0.4) (layers "F.Cu" "B.Cu") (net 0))
 (segment (start 151.13 80.01) (end 149.86 81.28) (width 0.15) (layer "B.Cu") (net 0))
 (segment (start 148.59 82.55) (end 160.02 82.55) (width 0.15) (layer "B.Cu") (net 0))
 (segment (start 132.08 86.36) (end 129.54 83.82) (width 0.15) (layer "B.Cu") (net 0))
 (segment (start 160.02 80.01) (end 151.13 80.01) (width 0.15) (layer "B.Cu") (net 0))
 (segment (start 111.76 83.82) (end 109.22 86.36) (width 0.15) (layer "B.Cu") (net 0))
 (segment (start 152.4 73.66) (end 154.94 73.66) (width 0.15) (layer "B.Cu") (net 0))
 (segment (start 158.75 77.47) (end 160.02 77.47) (width 0.15) (layer "B.Cu") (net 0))
 (segment (start 111.76 76.2) (end 99.06 88.9) (width 0.15) (layer "B.Cu") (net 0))
 (segment (start 149.86 71.12) (end 152.4 73.66) (width 0.15) (layer "B.Cu") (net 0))
 (segment (start 144.78 78.74) (end 148.59 82.55) (width 0.15) (layer "B.Cu") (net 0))
 (segment (start 142.24 102.87) (end 138.43 102.87) (width 0.15) (layer "B.Cu") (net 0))
 (segment (start 144.78 73.66) (end 101.6 73.66) (width 0.15) (layer "B.Cu") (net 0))
 (segment (start 101.6 73.66) (end 99.06 76.2) (width 0.15) (layer "B.Cu") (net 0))
 (segment (start 125.3 93.98) (end 118.8 87.48) (width 0.15) (layer "B.Cu") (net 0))
 (segment (start 109.22 86.36) (end 104.14 86.36) (width 0.15) (layer "B.Cu") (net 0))
 (segment (start 138.43 102.87) (end 129.54 93.98) (width 0.15) (layer "B.Cu") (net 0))
 (segment (start 129.54 93.98) (end 125.3 93.98) (width 0.15) (layer "B.Cu") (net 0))
 (segment (start 144.78 71.12) (end 144.78 78.74) (width 0.15) (layer "B.Cu") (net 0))
 (segment (start 154.94 73.66) (end 158.75 77.47) (width 0.15) (layer "B.Cu") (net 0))
 (segment (start 129.54 83.82) (end 111.76 83.82) (width 0.15) (layer "B.Cu") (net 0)))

